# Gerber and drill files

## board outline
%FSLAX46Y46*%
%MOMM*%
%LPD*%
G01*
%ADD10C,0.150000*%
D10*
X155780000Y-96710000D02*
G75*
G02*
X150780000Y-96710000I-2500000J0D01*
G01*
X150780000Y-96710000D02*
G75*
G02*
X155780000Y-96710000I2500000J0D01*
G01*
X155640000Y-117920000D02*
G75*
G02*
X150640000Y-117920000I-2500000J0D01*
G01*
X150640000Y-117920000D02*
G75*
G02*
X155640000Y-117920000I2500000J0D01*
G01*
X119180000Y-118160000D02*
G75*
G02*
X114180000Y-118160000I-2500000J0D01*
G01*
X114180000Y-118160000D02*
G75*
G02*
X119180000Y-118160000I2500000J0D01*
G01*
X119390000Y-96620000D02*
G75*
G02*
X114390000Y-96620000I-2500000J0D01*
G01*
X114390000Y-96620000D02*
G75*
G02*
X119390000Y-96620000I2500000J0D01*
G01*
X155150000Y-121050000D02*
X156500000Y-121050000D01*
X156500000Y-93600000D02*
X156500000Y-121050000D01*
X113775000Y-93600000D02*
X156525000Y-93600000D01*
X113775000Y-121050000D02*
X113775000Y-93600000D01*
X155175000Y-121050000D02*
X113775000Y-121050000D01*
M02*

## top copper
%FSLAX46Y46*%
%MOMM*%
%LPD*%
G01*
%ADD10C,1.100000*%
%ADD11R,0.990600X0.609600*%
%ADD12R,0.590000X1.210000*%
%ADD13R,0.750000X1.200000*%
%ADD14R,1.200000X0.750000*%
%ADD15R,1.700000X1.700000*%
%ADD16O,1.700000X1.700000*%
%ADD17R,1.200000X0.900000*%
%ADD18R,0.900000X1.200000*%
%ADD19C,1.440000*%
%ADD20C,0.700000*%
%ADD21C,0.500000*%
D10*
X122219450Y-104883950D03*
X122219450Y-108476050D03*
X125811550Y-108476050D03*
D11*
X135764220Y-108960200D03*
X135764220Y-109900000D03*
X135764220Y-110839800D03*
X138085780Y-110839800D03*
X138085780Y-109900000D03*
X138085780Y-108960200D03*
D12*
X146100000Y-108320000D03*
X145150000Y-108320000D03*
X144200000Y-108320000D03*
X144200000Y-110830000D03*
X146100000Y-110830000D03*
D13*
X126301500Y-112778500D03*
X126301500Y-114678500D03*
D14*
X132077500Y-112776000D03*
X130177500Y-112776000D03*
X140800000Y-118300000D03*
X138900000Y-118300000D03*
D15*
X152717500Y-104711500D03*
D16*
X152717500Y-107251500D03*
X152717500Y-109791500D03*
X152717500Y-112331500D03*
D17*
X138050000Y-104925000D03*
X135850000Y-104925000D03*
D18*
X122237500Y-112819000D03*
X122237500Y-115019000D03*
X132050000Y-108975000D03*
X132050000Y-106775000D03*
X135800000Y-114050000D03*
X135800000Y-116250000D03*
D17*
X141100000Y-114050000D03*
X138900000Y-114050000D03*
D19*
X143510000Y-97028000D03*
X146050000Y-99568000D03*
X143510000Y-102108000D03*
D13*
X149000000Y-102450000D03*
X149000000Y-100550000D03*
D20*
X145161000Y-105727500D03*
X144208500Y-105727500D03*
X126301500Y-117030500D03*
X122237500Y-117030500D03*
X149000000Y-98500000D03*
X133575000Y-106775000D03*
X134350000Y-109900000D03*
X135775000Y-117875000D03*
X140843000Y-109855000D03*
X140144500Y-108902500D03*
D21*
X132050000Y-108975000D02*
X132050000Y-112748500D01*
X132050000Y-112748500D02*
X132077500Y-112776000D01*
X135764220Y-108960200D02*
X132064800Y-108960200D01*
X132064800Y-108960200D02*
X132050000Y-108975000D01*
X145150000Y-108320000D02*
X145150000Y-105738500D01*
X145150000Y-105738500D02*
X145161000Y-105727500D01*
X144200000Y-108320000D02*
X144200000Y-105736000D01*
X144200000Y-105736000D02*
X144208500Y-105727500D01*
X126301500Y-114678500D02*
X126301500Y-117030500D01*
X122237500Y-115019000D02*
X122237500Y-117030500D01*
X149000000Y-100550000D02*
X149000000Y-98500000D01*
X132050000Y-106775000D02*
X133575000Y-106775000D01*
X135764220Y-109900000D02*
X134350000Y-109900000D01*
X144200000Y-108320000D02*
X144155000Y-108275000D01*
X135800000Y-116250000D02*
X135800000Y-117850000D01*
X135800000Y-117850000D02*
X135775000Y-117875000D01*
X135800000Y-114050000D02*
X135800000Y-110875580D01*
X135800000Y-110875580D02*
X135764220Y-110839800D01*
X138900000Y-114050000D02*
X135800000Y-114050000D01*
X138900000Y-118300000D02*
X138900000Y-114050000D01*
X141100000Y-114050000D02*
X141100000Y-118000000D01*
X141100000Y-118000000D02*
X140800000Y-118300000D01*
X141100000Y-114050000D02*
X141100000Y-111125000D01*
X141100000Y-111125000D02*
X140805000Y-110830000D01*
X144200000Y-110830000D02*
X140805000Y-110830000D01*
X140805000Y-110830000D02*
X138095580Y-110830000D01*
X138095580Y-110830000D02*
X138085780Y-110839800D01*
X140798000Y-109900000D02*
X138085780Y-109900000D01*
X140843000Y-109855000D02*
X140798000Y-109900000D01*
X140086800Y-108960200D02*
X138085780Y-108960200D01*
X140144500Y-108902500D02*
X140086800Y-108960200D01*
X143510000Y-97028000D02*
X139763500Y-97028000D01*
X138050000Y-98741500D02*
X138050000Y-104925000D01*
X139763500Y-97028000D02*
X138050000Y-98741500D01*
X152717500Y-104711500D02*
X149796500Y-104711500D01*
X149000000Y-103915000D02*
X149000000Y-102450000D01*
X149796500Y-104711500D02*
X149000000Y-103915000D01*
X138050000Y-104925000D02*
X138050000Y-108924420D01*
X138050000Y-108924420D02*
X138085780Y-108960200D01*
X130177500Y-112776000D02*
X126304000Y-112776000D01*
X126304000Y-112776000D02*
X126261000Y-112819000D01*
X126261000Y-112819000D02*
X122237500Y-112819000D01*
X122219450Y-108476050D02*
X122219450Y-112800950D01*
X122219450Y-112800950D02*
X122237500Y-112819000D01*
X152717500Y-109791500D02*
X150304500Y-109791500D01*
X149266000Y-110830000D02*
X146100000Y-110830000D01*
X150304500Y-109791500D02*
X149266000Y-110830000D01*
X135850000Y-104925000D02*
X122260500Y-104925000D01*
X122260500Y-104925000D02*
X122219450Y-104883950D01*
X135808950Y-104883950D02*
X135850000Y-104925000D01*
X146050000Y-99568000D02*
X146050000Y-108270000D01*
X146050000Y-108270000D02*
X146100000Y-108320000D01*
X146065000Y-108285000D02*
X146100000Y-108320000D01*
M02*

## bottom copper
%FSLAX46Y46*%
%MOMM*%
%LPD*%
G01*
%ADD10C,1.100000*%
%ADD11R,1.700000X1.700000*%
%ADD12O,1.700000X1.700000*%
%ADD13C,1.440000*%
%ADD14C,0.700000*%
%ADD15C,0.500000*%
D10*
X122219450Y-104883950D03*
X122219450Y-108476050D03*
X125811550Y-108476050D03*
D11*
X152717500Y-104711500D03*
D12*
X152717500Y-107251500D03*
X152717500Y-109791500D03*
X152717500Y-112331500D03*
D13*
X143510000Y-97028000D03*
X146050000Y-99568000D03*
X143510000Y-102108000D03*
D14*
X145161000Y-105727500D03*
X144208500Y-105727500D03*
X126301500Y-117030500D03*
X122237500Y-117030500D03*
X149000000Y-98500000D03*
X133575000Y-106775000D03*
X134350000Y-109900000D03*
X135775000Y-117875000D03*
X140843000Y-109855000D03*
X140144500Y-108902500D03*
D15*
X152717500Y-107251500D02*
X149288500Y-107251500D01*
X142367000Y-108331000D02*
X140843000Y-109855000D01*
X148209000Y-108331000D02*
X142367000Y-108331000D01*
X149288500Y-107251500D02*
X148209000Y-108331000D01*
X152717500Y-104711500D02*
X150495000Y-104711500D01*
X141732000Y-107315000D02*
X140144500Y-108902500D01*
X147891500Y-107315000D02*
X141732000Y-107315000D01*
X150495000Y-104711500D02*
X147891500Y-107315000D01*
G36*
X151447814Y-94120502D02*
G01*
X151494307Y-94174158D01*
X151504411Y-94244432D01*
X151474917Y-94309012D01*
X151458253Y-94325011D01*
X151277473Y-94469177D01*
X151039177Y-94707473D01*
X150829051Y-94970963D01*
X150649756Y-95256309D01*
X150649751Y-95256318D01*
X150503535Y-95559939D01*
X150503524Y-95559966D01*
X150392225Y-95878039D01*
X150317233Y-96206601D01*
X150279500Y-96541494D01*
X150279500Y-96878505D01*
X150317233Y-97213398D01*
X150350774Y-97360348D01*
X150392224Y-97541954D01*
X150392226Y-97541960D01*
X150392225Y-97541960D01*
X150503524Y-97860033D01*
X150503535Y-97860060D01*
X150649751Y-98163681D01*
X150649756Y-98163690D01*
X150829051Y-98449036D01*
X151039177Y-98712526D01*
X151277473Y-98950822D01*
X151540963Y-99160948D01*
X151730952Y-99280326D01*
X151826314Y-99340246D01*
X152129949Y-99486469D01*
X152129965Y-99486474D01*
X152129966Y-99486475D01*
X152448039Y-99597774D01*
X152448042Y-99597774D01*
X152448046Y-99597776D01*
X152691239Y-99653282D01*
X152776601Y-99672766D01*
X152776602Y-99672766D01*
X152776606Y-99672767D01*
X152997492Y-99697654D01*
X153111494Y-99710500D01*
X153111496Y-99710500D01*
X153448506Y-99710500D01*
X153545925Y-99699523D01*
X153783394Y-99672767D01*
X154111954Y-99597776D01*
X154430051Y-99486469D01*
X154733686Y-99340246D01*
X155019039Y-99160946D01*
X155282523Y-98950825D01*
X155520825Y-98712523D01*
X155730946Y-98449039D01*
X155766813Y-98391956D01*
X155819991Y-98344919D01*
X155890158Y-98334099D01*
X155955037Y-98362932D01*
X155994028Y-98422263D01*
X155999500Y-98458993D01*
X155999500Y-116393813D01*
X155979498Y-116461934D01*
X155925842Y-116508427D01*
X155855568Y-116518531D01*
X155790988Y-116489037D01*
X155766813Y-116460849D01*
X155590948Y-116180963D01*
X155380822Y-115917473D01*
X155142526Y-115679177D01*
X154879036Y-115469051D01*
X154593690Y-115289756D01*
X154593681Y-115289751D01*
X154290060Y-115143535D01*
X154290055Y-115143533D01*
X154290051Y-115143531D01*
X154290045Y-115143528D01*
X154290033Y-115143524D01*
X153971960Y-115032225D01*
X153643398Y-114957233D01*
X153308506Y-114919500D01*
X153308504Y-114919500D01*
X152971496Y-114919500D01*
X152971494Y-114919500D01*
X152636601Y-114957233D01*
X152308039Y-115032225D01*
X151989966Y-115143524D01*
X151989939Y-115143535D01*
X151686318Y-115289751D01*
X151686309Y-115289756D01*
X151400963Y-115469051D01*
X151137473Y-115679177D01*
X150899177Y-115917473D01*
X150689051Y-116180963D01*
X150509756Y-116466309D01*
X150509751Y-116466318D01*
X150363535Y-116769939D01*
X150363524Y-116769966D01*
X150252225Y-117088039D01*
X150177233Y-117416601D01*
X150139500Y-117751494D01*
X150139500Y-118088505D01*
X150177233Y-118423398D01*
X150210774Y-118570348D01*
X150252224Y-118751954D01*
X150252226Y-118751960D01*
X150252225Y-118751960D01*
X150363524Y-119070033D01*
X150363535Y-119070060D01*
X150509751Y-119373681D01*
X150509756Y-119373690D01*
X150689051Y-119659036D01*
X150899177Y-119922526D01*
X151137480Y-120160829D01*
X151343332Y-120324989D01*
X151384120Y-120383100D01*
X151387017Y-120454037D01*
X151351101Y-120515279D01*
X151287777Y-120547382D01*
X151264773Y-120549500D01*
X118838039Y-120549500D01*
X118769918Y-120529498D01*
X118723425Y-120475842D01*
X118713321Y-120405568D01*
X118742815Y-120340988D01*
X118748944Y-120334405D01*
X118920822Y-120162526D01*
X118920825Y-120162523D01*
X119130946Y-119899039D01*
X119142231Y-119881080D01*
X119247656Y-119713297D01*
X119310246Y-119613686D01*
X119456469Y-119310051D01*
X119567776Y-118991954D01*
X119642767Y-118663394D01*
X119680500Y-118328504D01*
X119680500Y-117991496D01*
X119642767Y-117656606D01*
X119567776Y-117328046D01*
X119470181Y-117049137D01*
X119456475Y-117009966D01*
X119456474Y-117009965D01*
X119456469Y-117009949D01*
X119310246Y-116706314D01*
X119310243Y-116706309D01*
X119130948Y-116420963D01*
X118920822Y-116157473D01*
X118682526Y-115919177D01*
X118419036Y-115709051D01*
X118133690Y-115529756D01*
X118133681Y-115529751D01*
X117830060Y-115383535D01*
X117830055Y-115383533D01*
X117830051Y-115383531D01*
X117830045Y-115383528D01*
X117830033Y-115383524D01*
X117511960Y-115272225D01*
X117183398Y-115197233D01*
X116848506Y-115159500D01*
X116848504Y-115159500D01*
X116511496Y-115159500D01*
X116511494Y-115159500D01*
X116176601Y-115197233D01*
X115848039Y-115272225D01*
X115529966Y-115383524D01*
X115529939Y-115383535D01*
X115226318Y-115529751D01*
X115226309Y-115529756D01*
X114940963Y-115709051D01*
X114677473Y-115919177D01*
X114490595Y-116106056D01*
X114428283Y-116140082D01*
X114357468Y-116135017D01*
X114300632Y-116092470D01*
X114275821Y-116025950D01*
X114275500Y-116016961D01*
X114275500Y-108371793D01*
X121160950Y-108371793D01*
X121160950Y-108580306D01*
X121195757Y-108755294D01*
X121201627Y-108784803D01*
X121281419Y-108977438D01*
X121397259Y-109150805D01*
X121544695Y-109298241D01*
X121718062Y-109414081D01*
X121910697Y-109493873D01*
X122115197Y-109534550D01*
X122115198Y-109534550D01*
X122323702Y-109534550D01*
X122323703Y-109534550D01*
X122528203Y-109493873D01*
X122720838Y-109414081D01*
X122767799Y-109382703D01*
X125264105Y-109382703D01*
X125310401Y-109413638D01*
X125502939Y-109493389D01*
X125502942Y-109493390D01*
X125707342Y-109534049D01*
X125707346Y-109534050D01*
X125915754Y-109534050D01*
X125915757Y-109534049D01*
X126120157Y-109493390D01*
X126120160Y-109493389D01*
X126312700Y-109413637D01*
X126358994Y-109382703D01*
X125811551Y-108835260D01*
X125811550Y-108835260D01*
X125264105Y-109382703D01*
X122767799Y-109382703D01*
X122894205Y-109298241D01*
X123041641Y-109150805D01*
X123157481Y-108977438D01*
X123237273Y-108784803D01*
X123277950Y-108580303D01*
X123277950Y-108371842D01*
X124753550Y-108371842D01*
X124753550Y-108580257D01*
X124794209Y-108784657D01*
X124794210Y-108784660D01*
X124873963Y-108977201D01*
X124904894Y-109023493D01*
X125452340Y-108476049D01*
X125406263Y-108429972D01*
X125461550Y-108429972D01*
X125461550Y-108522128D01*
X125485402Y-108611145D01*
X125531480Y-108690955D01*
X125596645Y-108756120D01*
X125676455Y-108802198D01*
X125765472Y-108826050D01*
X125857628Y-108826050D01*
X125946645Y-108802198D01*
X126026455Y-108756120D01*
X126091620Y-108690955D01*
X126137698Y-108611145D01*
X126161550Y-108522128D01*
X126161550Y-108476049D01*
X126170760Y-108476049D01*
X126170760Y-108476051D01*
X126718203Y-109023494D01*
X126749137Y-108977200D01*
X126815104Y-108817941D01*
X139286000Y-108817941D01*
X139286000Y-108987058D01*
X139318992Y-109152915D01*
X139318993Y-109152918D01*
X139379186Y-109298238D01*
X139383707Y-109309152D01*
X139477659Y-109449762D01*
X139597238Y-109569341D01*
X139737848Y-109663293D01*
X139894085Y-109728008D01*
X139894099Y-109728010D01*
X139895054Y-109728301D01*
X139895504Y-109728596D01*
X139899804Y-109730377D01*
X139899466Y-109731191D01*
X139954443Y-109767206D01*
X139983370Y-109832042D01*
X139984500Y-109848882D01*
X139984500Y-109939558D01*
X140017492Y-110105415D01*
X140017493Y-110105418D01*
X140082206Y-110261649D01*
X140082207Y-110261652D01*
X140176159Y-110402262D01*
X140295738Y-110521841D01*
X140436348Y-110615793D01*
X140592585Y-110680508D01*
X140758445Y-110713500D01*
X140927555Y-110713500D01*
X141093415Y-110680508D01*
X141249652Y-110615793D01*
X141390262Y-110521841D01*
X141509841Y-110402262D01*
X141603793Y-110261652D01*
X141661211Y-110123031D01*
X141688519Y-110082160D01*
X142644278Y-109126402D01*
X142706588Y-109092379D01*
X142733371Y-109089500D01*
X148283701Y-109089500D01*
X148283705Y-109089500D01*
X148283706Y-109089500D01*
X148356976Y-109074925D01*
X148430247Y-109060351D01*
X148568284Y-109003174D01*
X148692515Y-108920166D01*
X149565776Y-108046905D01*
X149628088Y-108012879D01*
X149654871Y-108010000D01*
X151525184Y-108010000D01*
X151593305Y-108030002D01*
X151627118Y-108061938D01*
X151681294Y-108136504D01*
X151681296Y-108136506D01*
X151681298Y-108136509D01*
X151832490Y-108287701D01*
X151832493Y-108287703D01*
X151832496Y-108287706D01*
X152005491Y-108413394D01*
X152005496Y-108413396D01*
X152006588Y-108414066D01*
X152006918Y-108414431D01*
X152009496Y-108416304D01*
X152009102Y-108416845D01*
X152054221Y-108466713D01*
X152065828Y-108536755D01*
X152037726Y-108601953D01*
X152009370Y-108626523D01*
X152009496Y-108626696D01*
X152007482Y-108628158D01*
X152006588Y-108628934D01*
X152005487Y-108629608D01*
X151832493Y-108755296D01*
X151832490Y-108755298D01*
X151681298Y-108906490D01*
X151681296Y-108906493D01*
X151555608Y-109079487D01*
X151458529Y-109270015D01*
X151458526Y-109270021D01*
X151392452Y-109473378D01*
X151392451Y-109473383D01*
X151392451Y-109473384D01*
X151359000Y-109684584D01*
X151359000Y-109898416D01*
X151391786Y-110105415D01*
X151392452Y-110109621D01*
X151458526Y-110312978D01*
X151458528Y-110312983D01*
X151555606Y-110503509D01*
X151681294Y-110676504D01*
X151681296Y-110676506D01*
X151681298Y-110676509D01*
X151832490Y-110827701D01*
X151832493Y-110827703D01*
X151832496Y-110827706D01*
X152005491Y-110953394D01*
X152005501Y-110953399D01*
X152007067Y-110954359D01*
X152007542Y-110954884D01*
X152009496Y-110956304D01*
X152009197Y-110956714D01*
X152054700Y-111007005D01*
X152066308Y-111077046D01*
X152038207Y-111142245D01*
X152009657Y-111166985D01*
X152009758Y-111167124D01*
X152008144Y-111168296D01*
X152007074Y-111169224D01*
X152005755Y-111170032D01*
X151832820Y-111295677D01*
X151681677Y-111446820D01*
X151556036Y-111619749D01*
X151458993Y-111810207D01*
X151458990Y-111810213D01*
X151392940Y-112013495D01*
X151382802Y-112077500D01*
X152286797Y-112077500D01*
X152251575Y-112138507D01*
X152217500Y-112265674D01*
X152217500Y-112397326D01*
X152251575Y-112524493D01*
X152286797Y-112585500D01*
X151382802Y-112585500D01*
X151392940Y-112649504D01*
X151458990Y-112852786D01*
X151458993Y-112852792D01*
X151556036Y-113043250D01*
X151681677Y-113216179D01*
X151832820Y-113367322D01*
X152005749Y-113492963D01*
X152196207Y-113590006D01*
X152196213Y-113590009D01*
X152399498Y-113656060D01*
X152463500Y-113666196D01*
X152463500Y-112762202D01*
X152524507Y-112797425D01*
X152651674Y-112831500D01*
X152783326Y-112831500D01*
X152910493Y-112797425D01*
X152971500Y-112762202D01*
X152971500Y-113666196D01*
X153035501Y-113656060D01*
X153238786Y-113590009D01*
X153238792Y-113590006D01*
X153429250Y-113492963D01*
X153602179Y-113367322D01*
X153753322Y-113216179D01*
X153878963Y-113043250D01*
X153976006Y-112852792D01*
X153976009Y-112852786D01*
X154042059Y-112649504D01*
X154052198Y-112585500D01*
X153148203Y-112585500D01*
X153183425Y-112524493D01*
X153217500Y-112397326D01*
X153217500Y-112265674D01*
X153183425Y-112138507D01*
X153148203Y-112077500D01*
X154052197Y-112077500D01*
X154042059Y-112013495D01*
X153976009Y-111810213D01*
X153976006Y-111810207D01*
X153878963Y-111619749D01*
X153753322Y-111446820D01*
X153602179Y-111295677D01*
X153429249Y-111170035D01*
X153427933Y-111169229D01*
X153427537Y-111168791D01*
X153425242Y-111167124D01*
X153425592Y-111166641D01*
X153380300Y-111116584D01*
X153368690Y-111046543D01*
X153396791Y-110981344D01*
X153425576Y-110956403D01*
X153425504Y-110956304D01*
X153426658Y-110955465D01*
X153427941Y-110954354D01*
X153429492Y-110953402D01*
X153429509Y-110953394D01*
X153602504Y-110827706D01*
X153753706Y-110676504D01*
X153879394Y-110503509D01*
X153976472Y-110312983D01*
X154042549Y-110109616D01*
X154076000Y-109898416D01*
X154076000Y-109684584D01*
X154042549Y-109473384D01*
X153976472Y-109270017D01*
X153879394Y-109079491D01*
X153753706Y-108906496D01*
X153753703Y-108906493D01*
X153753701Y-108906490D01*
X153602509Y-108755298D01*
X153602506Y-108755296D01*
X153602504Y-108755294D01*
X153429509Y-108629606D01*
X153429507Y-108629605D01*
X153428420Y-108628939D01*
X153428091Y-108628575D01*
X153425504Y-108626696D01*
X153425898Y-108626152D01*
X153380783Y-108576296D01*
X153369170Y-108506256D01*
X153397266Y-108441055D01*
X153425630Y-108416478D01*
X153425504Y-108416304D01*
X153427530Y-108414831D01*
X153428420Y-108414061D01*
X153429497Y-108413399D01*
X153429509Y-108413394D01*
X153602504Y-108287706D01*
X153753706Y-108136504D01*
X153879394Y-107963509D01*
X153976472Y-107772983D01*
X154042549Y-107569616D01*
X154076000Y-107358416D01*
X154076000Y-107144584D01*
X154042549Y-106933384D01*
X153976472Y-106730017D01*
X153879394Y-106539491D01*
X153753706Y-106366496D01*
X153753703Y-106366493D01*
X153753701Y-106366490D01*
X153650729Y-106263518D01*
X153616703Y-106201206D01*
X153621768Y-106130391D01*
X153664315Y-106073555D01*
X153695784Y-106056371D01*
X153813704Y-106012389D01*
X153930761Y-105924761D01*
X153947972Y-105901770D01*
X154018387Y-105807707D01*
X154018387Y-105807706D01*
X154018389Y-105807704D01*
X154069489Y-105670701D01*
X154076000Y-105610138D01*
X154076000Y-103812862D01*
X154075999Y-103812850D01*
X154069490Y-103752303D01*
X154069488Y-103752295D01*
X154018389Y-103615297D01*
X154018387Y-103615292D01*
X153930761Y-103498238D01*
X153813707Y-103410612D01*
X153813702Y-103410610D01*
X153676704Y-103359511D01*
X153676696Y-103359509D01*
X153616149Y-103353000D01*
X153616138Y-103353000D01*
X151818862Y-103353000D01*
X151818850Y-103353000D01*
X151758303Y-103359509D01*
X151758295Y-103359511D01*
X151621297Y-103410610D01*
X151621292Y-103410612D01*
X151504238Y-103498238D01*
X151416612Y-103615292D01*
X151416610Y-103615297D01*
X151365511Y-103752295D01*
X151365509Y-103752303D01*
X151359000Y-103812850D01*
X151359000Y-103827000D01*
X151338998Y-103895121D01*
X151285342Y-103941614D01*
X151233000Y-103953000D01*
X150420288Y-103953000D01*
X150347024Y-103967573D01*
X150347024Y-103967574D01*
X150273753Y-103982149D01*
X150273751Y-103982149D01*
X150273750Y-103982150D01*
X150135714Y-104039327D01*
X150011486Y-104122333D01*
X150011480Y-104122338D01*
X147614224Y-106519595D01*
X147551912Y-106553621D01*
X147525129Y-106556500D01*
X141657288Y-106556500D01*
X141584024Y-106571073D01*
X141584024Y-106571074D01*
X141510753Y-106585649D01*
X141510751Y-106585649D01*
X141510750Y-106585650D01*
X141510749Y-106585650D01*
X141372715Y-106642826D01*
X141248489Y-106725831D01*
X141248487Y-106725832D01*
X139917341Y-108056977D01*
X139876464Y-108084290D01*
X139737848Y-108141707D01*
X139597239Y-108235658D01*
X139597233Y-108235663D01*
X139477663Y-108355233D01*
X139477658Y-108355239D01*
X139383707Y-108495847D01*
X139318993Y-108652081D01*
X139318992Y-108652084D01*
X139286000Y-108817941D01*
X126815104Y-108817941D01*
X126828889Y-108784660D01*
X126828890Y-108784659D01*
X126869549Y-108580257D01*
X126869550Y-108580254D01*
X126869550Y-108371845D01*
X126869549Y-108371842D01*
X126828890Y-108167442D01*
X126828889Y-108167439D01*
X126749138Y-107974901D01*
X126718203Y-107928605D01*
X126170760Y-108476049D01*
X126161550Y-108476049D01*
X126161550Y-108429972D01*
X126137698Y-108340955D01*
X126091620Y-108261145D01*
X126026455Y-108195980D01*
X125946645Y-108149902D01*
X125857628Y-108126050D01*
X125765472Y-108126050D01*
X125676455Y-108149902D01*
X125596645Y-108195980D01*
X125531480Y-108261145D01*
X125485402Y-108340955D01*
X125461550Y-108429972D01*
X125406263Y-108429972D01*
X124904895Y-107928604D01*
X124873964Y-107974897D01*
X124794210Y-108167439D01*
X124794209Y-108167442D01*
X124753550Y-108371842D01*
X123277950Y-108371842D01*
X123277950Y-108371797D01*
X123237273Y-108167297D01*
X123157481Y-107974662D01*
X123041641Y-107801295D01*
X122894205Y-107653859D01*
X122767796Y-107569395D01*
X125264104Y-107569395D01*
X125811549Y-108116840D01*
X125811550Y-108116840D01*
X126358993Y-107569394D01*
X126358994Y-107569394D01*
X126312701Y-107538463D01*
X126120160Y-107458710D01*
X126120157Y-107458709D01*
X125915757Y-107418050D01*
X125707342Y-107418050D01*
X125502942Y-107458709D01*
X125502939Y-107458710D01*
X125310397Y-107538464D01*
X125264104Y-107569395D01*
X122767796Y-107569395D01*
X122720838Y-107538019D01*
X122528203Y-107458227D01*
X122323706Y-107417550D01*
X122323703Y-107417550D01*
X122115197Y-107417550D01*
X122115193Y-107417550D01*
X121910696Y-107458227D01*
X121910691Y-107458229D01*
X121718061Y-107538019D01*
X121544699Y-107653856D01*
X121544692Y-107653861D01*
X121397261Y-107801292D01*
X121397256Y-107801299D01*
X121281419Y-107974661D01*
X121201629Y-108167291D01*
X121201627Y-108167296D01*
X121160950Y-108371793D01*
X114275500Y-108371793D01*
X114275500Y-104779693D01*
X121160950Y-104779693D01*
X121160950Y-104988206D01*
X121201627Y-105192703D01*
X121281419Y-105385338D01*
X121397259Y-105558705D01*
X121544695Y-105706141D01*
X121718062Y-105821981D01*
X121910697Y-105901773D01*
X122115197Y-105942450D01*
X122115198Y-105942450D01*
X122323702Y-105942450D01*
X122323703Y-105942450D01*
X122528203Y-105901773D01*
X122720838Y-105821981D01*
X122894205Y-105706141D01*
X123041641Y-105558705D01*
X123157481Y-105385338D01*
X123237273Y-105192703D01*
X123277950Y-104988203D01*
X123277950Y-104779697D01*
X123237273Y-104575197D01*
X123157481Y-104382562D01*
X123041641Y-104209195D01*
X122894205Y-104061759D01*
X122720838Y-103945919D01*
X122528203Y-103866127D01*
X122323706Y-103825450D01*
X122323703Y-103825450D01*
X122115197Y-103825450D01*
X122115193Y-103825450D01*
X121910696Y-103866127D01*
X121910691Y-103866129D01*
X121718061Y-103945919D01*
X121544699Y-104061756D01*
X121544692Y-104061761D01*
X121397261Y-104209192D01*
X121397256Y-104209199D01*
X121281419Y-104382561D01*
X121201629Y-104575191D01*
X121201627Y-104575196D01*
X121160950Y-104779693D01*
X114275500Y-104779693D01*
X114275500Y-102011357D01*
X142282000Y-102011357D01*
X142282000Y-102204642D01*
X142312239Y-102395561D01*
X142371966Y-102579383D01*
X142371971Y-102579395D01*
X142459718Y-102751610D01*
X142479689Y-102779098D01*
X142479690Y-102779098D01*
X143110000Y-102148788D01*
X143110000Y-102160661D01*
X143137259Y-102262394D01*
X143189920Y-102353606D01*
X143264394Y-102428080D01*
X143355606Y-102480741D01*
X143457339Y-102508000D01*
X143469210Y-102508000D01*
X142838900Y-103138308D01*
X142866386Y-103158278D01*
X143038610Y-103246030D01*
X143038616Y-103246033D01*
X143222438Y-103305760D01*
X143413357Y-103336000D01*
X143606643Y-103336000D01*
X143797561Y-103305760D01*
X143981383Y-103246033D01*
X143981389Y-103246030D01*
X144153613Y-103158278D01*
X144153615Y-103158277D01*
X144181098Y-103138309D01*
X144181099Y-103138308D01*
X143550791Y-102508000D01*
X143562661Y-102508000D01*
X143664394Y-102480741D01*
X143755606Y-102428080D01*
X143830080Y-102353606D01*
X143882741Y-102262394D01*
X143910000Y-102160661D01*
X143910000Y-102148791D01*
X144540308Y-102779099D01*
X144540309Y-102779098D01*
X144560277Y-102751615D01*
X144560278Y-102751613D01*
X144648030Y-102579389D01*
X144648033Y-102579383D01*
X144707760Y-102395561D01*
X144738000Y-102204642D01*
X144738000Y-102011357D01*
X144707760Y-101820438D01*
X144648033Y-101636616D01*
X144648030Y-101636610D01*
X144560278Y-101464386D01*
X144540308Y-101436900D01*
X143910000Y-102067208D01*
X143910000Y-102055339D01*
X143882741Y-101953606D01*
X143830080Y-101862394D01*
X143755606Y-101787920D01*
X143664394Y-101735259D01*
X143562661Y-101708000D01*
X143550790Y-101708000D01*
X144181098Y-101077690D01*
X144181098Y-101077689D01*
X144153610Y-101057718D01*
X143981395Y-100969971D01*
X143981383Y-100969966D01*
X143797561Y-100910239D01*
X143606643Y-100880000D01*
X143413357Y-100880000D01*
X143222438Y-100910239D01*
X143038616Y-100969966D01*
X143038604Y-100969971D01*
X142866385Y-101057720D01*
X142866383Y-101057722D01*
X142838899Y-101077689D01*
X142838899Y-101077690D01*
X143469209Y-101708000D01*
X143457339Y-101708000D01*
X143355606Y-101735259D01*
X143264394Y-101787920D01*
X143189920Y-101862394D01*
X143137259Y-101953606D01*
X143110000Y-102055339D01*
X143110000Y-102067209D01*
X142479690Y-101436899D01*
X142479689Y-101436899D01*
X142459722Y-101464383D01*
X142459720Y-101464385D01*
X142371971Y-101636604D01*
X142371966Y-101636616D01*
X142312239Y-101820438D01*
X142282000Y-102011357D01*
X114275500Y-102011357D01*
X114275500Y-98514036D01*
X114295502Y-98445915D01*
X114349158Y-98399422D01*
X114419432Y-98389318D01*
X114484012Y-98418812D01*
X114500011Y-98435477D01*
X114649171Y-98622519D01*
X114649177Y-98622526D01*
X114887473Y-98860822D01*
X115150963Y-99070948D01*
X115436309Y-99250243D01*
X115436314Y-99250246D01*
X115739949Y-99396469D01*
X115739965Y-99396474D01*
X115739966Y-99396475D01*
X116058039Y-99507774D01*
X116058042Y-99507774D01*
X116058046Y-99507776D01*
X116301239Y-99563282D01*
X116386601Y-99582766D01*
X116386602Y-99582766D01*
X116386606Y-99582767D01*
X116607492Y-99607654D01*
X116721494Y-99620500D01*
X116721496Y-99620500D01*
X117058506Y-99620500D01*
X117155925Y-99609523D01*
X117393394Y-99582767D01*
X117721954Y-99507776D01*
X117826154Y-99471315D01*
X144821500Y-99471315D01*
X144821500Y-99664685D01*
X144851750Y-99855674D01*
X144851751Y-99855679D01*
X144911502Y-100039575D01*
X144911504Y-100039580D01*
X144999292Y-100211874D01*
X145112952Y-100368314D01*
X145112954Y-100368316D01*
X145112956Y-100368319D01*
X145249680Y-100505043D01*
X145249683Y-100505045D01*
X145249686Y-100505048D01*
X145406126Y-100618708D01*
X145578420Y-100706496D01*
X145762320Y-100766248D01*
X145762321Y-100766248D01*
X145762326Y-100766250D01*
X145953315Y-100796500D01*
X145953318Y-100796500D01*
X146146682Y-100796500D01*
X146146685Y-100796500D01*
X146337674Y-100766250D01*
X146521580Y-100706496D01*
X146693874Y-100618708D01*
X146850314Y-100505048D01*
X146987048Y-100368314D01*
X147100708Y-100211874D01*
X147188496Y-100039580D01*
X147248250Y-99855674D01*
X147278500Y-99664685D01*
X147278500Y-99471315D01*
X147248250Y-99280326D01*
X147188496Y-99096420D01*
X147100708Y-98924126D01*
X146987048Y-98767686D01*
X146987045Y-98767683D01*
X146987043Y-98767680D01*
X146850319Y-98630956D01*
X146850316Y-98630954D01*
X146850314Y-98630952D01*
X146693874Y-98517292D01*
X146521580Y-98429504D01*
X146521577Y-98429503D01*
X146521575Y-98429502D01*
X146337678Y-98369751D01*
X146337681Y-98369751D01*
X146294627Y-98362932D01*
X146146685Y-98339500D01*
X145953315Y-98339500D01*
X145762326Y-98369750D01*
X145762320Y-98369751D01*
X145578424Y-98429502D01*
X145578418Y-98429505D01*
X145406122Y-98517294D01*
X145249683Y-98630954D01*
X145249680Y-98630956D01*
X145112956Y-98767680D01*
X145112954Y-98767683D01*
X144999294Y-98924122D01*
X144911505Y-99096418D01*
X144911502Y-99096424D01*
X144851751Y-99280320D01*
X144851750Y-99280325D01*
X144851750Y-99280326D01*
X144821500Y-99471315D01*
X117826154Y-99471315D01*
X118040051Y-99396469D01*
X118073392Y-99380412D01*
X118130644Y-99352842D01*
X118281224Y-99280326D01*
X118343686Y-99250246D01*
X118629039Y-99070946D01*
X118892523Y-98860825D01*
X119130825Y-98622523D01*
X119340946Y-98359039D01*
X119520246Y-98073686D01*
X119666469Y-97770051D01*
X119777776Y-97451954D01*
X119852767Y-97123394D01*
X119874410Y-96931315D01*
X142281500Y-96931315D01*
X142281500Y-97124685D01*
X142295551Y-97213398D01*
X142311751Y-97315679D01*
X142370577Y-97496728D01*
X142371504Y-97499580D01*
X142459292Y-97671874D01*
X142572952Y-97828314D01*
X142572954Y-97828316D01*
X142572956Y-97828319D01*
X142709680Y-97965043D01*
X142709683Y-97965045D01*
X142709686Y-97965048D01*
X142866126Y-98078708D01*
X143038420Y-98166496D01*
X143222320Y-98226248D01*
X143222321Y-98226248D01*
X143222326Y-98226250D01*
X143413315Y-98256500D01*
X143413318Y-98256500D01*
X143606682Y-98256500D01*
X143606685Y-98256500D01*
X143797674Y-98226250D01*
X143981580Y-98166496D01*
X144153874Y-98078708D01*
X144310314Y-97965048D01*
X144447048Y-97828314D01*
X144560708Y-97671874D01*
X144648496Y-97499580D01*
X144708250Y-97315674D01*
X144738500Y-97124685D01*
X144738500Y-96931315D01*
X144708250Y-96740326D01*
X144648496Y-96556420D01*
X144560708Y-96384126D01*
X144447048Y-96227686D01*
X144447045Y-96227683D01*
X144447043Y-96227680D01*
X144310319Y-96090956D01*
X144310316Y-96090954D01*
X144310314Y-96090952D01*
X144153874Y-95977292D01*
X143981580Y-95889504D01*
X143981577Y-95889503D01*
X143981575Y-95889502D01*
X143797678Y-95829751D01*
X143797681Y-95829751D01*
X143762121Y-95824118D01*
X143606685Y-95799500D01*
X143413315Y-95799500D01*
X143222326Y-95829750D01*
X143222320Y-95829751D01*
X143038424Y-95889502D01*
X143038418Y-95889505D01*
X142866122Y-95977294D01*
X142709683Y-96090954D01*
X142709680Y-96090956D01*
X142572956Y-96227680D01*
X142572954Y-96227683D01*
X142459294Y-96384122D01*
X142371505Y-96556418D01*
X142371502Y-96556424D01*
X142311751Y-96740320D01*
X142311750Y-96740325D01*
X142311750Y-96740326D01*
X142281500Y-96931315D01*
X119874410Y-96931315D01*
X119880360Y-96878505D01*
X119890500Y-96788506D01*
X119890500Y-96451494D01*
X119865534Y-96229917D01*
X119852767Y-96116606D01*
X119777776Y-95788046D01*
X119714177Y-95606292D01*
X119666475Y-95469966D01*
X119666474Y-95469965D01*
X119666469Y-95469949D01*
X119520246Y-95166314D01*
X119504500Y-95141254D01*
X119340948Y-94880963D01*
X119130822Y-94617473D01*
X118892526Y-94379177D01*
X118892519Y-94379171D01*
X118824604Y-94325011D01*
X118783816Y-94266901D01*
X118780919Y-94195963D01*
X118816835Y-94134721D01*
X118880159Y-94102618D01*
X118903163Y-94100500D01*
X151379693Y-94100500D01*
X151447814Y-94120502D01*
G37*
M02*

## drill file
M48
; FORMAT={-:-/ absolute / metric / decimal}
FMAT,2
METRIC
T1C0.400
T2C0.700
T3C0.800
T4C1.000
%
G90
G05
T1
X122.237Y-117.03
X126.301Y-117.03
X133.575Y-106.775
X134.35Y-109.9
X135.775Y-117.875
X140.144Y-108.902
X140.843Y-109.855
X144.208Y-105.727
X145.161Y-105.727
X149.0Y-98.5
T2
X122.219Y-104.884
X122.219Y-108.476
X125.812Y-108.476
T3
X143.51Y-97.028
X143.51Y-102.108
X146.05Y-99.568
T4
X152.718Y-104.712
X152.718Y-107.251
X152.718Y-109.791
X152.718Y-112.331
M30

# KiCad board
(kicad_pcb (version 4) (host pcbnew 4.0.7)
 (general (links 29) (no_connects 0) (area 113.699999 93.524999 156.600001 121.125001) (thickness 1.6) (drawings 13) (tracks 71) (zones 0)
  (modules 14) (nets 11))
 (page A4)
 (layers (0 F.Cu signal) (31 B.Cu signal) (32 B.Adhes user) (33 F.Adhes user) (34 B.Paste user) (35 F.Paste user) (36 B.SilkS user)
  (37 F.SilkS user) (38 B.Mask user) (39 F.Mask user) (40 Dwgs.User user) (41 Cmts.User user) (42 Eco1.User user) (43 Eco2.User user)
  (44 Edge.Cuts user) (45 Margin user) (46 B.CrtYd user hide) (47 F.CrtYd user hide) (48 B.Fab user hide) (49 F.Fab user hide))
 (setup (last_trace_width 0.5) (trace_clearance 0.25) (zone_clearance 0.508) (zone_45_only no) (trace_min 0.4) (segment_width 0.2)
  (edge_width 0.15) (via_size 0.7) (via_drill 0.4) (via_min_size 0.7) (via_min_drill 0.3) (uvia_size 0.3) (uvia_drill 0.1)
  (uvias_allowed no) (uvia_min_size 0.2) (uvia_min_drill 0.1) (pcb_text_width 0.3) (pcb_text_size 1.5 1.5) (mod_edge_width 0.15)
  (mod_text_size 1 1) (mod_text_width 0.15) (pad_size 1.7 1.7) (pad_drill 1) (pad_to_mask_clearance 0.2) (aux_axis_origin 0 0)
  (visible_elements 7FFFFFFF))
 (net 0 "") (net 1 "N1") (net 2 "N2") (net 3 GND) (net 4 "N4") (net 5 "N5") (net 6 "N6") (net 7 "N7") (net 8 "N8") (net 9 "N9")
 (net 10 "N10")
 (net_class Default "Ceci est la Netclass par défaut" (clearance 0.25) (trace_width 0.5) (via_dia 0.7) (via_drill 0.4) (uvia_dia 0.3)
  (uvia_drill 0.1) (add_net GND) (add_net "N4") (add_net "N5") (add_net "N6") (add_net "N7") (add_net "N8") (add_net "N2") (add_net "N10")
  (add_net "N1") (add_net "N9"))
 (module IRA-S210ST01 (layer F.Cu) (at 124.0155 106.68 270)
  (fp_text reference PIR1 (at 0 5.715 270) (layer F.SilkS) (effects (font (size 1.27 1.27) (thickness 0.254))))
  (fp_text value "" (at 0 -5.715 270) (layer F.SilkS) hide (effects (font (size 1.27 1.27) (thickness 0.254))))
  (pad 1 thru_hole circle (at -1.79605 1.79605) (size 1.1 1.1) (drill 0.7) (layers *.Cu *.Mask F.SilkS) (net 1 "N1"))
  (pad 2 thru_hole circle (at 1.79605 1.79605) (size 1.1 1.1) (drill 0.7) (layers *.Cu *.Mask F.SilkS) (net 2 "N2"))
  (pad 3 thru_hole circle (at 1.79605 -1.79605) (size 1.1 1.1) (drill 0.7) (layers *.Cu *.Mask F.SilkS) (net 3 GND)))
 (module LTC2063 (layer F.Cu) (at 136.925 109.9)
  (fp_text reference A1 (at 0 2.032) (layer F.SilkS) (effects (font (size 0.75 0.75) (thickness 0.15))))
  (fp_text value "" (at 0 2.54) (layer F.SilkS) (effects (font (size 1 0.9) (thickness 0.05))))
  (pad 1 smd rect (at -1.16078 -0.9398) (size 0.9906 0.6096) (layers F.Cu F.Paste F.Mask) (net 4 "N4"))
  (pad 2 smd rect (at -1.16078 0) (size 0.9906 0.6096) (layers F.Cu F.Paste F.Mask) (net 3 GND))
  (pad 3 smd rect (at -1.16078 0.9398) (size 0.9906 0.6096) (layers F.Cu F.Paste F.Mask) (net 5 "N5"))
  (pad 4 smd rect (at 1.16078 0.9398) (size 0.9906 0.6096) (layers F.Cu F.Paste F.Mask) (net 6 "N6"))
  (pad 5 smd rect (at 1.16078 0) (size 0.9906 0.6096) (layers F.Cu F.Paste F.Mask) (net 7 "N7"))
  (pad 6 smd rect (at 1.16078 -0.9398) (size 0.9906 0.6096) (layers F.Cu F.Paste F.Mask) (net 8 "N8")))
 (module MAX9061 (layer F.Cu) (at 145.15 109.575 270)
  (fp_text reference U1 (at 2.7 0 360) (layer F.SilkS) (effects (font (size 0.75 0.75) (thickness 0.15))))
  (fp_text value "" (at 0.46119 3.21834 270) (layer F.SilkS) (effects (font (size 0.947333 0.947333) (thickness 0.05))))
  (pad 1 smd rect (at -1.255 -0.95 90) (size 1.21 0.59) (layers F.Cu F.Paste F.Mask) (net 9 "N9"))
  (pad 2 smd rect (at -1.255 0 90) (size 1.21 0.59) (layers F.Cu F.Paste F.Mask) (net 3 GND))
  (pad 3 smd rect (at -1.255 0.95 90) (size 1.21 0.59) (layers F.Cu F.Paste F.Mask) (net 3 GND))
  (pad 4 smd rect (at 1.255 0.95 270) (size 1.21 0.59) (layers F.Cu F.Paste F.Mask) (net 6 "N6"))
  (pad 5 smd rect (at 1.255 -0.95 270) (size 1.21 0.59) (layers F.Cu F.Paste F.Mask) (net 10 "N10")))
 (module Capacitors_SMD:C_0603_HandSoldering (layer F.Cu) (at 126.3015 113.7285 270)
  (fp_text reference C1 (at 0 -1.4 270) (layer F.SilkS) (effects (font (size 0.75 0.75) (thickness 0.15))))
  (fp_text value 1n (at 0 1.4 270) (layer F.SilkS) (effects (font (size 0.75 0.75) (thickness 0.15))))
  (pad 1 smd rect (at -0.95 0 270) (size 1.2 0.75) (layers F.Cu F.Paste F.Mask) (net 2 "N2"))
  (pad 2 smd rect (at 0.95 0 270) (size 1.2 0.75) (layers F.Cu F.Paste F.Mask) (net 3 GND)))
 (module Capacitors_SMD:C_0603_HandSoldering (layer F.Cu) (at 131.1275 112.776 180)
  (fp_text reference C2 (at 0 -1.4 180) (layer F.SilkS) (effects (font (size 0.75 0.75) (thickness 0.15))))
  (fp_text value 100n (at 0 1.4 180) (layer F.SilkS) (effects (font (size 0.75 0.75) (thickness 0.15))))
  (pad 1 smd rect (at -0.95 0 180) (size 1.2 0.75) (layers F.Cu F.Paste F.Mask) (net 4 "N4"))
  (pad 2 smd rect (at 0.95 0 180) (size 1.2 0.75) (layers F.Cu F.Paste F.Mask) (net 2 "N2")))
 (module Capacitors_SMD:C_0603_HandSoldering (layer F.Cu) (at 139.85 118.3 180)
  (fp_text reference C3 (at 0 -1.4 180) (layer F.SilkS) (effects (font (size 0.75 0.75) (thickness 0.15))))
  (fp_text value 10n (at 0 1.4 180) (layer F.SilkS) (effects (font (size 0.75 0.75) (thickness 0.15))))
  (pad 1 smd rect (at -0.95 0 180) (size 1.2 0.75) (layers F.Cu F.Paste F.Mask) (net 6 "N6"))
  (pad 2 smd rect (at 0.95 0 180) (size 1.2 0.75) (layers F.Cu F.Paste F.Mask) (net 5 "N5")))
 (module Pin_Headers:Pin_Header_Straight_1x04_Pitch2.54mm (layer F.Cu) (at 152.7175 104.7115)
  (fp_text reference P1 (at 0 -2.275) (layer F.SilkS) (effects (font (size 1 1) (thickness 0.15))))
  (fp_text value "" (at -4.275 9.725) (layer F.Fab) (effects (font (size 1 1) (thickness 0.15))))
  (pad 1 thru_hole rect (at 0 0) (size 1.7 1.7) (drill 1) (layers *.Cu *.Mask) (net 8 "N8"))
  (pad 2 thru_hole oval (at 0 2.54) (size 1.7 1.7) (drill 1) (layers *.Cu *.Mask) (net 7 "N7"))
  (pad 3 thru_hole oval (at 0 5.08) (size 1.7 1.7) (drill 1) (layers *.Cu *.Mask) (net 10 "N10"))
  (pad 4 thru_hole oval (at 0 7.62) (size 1.7 1.7) (drill 1) (layers *.Cu *.Mask) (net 3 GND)))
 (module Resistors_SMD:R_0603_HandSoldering (layer F.Cu) (at 136.95 104.925 180)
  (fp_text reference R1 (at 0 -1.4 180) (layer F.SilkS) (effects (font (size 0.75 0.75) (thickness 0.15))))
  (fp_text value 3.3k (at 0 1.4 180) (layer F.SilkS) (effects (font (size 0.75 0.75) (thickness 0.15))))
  (pad 1 smd rect (at -1.1 0 180) (size 1.2 0.9) (layers F.Cu F.Paste F.Mask) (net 8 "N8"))
  (pad 2 smd rect (at 1.1 0 180) (size 1.2 0.9) (layers F.Cu F.Paste F.Mask) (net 1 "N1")))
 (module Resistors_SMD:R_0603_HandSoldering (layer F.Cu) (at 122.2375 113.919 270)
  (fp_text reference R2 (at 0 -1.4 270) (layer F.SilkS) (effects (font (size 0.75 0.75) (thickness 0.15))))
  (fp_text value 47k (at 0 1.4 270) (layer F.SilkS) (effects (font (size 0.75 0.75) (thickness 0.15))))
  (pad 1 smd rect (at -1.1 0 270) (size 1.2 0.9) (layers F.Cu F.Paste F.Mask) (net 2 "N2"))
  (pad 2 smd rect (at 1.1 0 270) (size 1.2 0.9) (layers F.Cu F.Paste F.Mask) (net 3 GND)))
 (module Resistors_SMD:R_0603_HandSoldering (layer F.Cu) (at 132.05 107.875 90)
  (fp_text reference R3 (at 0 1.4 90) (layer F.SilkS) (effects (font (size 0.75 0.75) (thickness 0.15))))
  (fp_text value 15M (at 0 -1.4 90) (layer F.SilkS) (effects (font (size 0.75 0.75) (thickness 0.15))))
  (pad 1 smd rect (at -1.1 0 90) (size 1.2 0.9) (layers F.Cu F.Paste F.Mask) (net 4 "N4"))
  (pad 2 smd rect (at 1.1 0 90) (size 1.2 0.9) (layers F.Cu F.Paste F.Mask) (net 3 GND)))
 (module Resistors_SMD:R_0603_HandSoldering (layer F.Cu) (at 135.8 115.15 270)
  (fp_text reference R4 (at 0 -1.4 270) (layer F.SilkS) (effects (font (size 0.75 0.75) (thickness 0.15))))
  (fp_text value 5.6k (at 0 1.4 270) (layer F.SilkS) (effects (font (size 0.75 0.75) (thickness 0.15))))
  (pad 1 smd rect (at -1.1 0 270) (size 1.2 0.9) (layers F.Cu F.Paste F.Mask) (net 5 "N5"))
  (pad 2 smd rect (at 1.1 0 270) (size 1.2 0.9) (layers F.Cu F.Paste F.Mask) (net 3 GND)))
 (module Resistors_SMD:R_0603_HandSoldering (layer F.Cu) (at 140 114.05 180)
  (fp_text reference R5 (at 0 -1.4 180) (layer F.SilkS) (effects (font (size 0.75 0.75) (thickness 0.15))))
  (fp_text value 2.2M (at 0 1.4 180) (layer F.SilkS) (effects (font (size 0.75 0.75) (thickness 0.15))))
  (pad 1 smd rect (at -1.1 0 180) (size 1.2 0.9) (layers F.Cu F.Paste F.Mask) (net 6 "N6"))
  (pad 2 smd rect (at 1.1 0 180) (size 1.2 0.9) (layers F.Cu F.Paste F.Mask) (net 5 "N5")))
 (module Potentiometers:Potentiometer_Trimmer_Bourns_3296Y (layer F.Cu) (at 143.51 97.028 90)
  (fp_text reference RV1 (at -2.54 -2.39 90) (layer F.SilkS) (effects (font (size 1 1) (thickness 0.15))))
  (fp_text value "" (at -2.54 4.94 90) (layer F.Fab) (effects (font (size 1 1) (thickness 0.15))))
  (pad 1 thru_hole circle (at 0 0 90) (size 1.44 1.44) (drill 0.8) (layers *.Cu *.Mask) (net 8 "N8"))
  (pad 2 thru_hole circle (at -2.54 2.54 90) (size 1.44 1.44) (drill 0.8) (layers *.Cu *.Mask) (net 9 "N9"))
  (pad 3 thru_hole circle (at -5.08 0 90) (size 1.44 1.44) (drill 0.8) (layers *.Cu *.Mask) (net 3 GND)))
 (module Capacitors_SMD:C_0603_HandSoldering (layer F.Cu) (at 149 101.5 90)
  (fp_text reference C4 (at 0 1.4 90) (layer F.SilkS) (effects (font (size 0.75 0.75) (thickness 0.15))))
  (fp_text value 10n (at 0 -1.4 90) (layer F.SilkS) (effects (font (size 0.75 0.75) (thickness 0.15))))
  (pad 1 smd rect (at -0.95 0 90) (size 1.2 0.75) (layers F.Cu F.Paste F.Mask) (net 8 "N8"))
  (pad 2 smd rect (at 0.95 0 90) (size 1.2 0.75) (layers F.Cu F.Paste F.Mask) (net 3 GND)))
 (gr_circle (center 153.28 96.71) (end 155.78 96.71) (layer Edge.Cuts) (width 0.15))
 (gr_circle (center 153.14 117.92) (end 155.64 117.92) (layer Edge.Cuts) (width 0.15))
 (gr_circle (center 116.68 118.16) (end 119.18 118.16) (layer Edge.Cuts) (width 0.15))
 (gr_circle (center 116.89 96.62) (end 119.39 96.62) (layer Edge.Cuts) (width 0.15))
 (gr_line (start 155.15 121.05) (end 156.5 121.05) (angle 90) (layer Edge.Cuts) (width 0.15))
 (gr_line (start 156.5 93.6) (end 156.5 121.05) (angle 90) (layer Edge.Cuts) (width 0.15))
 (gr_line (start 113.775 93.6) (end 156.525 93.6) (angle 90) (layer Edge.Cuts) (width 0.15))
 (gr_line (start 113.775 121.05) (end 113.775 93.6) (angle 90) (layer Edge.Cuts) (width 0.15))
 (gr_line (start 155.175 121.05) (end 113.775 121.05) (angle 90) (layer Edge.Cuts) (width 0.15))
 (segment (start 132.05 108.975) (end 132.05 112.7485) (width 0.5) (layer F.Cu) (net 4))
 (segment (start 132.05 112.7485) (end 132.0775 112.776) (width 0.5) (layer F.Cu) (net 4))
 (segment (start 135.76422 108.9602) (end 132.0648 108.9602) (width 0.5) (layer F.Cu) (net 4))
 (segment (start 132.0648 108.9602) (end 132.05 108.975) (width 0.5) (layer F.Cu) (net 4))
 (segment (start 145.15 108.32) (end 145.15 105.7385) (width 0.5) (layer F.Cu) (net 3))
 (via (at 145.161 105.7275) (size 0.7) (drill 0.4) (layers F.Cu B.Cu) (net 3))
 (segment (start 145.15 105.7385) (end 145.161 105.7275) (width 0.5) (layer F.Cu) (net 3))
 (segment (start 144.2 108.32) (end 144.2 105.736) (width 0.5) (layer F.Cu) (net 3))
 (via (at 144.2085 105.7275) (size 0.7) (drill 0.4) (layers F.Cu B.Cu) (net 3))
 (segment (start 144.2 105.736) (end 144.2085 105.7275) (width 0.5) (layer F.Cu) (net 3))
 (segment (start 126.3015 114.6785) (end 126.3015 117.0305) (width 0.5) (layer F.Cu) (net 3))
 (via (at 126.3015 117.0305) (size 0.7) (drill 0.4) (layers F.Cu B.Cu) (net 3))
 (segment (start 122.2375 115.019) (end 122.2375 117.0305) (width 0.5) (layer F.Cu) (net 3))
 (via (at 122.2375 117.0305) (size 0.7) (drill 0.4) (layers F.Cu B.Cu) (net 3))
 (segment (start 149 100.55) (end 149 98.5) (width 0.5) (layer F.Cu) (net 3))
 (via (at 149 98.5) (size 0.7) (drill 0.4) (layers F.Cu B.Cu) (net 3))
 (segment (start 132.05 106.775) (end 133.575 106.775) (width 0.5) (layer F.Cu) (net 3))
 (via (at 133.575 106.775) (size 0.7) (drill 0.4) (layers F.Cu B.Cu) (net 3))
 (segment (start 135.76422 109.9) (end 134.35 109.9) (width 0.5) (layer F.Cu) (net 3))
 (via (at 134.35 109.9) (size 0.7) (drill 0.4) (layers F.Cu B.Cu) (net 3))
 (segment (start 144.2 108.32) (end 144.155 108.275) (width 0.5) (layer F.Cu) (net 3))
 (segment (start 135.8 116.25) (end 135.8 117.85) (width 0.5) (layer F.Cu) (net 3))
 (via (at 135.775 117.875) (size 0.7) (drill 0.4) (layers F.Cu B.Cu) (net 3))
 (segment (start 135.8 117.85) (end 135.775 117.875) (width 0.5) (layer F.Cu) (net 3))
 (segment (start 135.8 114.05) (end 135.8 110.87558) (width 0.5) (layer F.Cu) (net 5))
 (segment (start 135.8 110.87558) (end 135.76422 110.8398) (width 0.5) (layer F.Cu) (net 5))
 (segment (start 138.9 114.05) (end 135.8 114.05) (width 0.5) (layer F.Cu) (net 5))
 (segment (start 138.9 118.3) (end 138.9 114.05) (width 0.5) (layer F.Cu) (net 5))
 (segment (start 141.1 114.05) (end 141.1 118) (width 0.5) (layer F.Cu) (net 6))
 (segment (start 141.1 118) (end 140.8 118.3) (width 0.5) (layer F.Cu) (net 6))
 (segment (start 141.1 114.05) (end 141.1 111.125) (width 0.5) (layer F.Cu) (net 6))
 (segment (start 141.1 111.125) (end 140.805 110.83) (width 0.5) (layer F.Cu) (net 6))
 (segment (start 144.2 110.83) (end 140.805 110.83) (width 0.5) (layer F.Cu) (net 6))
 (segment (start 140.805 110.83) (end 138.09558 110.83) (width 0.5) (layer F.Cu) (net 6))
 (segment (start 138.09558 110.83) (end 138.08578 110.8398) (width 0.5) (layer F.Cu) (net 6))
 (segment (start 152.7175 107.2515) (end 149.2885 107.2515) (width 0.5) (layer B.Cu) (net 7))
 (segment (start 140.798 109.9) (end 138.08578 109.9) (width 0.5) (layer F.Cu) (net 7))
 (segment (start 140.843 109.855) (end 140.798 109.9) (width 0.5) (layer F.Cu) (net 7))
 (via (at 140.843 109.855) (size 0.7) (drill 0.4) (layers F.Cu B.Cu) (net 7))
 (segment (start 142.367 108.331) (end 140.843 109.855) (width 0.5) (layer B.Cu) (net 7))
 (segment (start 148.209 108.331) (end 142.367 108.331) (width 0.5) (layer B.Cu) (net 7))
 (segment (start 149.2885 107.2515) (end 148.209 108.331) (width 0.5) (layer B.Cu) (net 7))
 (segment (start 152.7175 104.7115) (end 150.495 104.7115) (width 0.5) (layer B.Cu) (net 8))
 (segment (start 140.0868 108.9602) (end 138.08578 108.9602) (width 0.5) (layer F.Cu) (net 8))
 (segment (start 140.1445 108.9025) (end 140.0868 108.9602) (width 0.5) (layer F.Cu) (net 8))
 (via (at 140.1445 108.9025) (size 0.7) (drill 0.4) (layers F.Cu B.Cu) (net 8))
 (segment (start 141.732 107.315) (end 140.1445 108.9025) (width 0.5) (layer B.Cu) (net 8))
 (segment (start 147.8915 107.315) (end 141.732 107.315) (width 0.5) (layer B.Cu) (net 8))
 (segment (start 150.495 104.7115) (end 147.8915 107.315) (width 0.5) (layer B.Cu) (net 8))
 (segment (start 143.51 97.028) (end 139.7635 97.028) (width 0.5) (layer F.Cu) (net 8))
 (segment (start 138.05 98.7415) (end 138.05 104.925) (width 0.5) (layer F.Cu) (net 8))
 (segment (start 139.7635 97.028) (end 138.05 98.7415) (width 0.5) (layer F.Cu) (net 8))
 (segment (start 152.7175 104.7115) (end 149.7965 104.7115) (width 0.5) (layer F.Cu) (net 8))
 (segment (start 149 103.915) (end 149 102.45) (width 0.5) (layer F.Cu) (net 8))
 (segment (start 149.7965 104.7115) (end 149 103.915) (width 0.5) (layer F.Cu) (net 8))
 (segment (start 138.05 104.925) (end 138.05 108.92442) (width 0.5) (layer F.Cu) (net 8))
 (segment (start 138.05 108.92442) (end 138.08578 108.9602) (width 0.5) (layer F.Cu) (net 8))
 (segment (start 130.1775 112.776) (end 126.304 112.776) (width 0.5) (layer F.Cu) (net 2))
 (segment (start 126.304 112.776) (end 126.261 112.819) (width 0.5) (layer F.Cu) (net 2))
 (segment (start 126.261 112.819) (end 122.2375 112.819) (width 0.5) (layer F.Cu) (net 2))
 (segment (start 122.21945 108.47605) (end 122.21945 112.80095) (width 0.5) (layer F.Cu) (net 2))
 (segment (start 122.21945 112.80095) (end 122.2375 112.819) (width 0.5) (layer F.Cu) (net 2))
 (segment (start 152.7175 109.7915) (end 150.3045 109.7915) (width 0.5) (layer F.Cu) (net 10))
 (segment (start 149.266 110.83) (end 146.1 110.83) (width 0.5) (layer F.Cu) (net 10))
 (segment (start 150.3045 109.7915) (end 149.266 110.83) (width 0.5) (layer F.Cu) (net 10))
 (segment (start 135.85 104.925) (end 122.2605 104.925) (width 0.5) (layer F.Cu) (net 1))
 (segment (start 122.2605 104.925) (end 122.21945 104.88395) (width 0.5) (layer F.Cu) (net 1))
 (segment (start 135.80895 104.88395) (end 135.85 104.925) (width 0.5) (layer F.Cu) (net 1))
 (segment (start 146.05 99.568) (end 146.05 108.27) (width 0.5) (layer F.Cu) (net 9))
 (segment (start 146.05 108.27) (end 146.1 108.32) (width 0.5) (layer F.Cu) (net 9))
 (segment (start 146.065 108.285) (end 146.1 108.32) (width 0.5) (layer F.Cu) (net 9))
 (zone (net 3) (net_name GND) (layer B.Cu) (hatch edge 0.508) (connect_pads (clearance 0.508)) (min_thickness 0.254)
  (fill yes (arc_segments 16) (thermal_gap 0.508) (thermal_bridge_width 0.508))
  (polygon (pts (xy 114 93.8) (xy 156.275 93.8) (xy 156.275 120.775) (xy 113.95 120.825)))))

